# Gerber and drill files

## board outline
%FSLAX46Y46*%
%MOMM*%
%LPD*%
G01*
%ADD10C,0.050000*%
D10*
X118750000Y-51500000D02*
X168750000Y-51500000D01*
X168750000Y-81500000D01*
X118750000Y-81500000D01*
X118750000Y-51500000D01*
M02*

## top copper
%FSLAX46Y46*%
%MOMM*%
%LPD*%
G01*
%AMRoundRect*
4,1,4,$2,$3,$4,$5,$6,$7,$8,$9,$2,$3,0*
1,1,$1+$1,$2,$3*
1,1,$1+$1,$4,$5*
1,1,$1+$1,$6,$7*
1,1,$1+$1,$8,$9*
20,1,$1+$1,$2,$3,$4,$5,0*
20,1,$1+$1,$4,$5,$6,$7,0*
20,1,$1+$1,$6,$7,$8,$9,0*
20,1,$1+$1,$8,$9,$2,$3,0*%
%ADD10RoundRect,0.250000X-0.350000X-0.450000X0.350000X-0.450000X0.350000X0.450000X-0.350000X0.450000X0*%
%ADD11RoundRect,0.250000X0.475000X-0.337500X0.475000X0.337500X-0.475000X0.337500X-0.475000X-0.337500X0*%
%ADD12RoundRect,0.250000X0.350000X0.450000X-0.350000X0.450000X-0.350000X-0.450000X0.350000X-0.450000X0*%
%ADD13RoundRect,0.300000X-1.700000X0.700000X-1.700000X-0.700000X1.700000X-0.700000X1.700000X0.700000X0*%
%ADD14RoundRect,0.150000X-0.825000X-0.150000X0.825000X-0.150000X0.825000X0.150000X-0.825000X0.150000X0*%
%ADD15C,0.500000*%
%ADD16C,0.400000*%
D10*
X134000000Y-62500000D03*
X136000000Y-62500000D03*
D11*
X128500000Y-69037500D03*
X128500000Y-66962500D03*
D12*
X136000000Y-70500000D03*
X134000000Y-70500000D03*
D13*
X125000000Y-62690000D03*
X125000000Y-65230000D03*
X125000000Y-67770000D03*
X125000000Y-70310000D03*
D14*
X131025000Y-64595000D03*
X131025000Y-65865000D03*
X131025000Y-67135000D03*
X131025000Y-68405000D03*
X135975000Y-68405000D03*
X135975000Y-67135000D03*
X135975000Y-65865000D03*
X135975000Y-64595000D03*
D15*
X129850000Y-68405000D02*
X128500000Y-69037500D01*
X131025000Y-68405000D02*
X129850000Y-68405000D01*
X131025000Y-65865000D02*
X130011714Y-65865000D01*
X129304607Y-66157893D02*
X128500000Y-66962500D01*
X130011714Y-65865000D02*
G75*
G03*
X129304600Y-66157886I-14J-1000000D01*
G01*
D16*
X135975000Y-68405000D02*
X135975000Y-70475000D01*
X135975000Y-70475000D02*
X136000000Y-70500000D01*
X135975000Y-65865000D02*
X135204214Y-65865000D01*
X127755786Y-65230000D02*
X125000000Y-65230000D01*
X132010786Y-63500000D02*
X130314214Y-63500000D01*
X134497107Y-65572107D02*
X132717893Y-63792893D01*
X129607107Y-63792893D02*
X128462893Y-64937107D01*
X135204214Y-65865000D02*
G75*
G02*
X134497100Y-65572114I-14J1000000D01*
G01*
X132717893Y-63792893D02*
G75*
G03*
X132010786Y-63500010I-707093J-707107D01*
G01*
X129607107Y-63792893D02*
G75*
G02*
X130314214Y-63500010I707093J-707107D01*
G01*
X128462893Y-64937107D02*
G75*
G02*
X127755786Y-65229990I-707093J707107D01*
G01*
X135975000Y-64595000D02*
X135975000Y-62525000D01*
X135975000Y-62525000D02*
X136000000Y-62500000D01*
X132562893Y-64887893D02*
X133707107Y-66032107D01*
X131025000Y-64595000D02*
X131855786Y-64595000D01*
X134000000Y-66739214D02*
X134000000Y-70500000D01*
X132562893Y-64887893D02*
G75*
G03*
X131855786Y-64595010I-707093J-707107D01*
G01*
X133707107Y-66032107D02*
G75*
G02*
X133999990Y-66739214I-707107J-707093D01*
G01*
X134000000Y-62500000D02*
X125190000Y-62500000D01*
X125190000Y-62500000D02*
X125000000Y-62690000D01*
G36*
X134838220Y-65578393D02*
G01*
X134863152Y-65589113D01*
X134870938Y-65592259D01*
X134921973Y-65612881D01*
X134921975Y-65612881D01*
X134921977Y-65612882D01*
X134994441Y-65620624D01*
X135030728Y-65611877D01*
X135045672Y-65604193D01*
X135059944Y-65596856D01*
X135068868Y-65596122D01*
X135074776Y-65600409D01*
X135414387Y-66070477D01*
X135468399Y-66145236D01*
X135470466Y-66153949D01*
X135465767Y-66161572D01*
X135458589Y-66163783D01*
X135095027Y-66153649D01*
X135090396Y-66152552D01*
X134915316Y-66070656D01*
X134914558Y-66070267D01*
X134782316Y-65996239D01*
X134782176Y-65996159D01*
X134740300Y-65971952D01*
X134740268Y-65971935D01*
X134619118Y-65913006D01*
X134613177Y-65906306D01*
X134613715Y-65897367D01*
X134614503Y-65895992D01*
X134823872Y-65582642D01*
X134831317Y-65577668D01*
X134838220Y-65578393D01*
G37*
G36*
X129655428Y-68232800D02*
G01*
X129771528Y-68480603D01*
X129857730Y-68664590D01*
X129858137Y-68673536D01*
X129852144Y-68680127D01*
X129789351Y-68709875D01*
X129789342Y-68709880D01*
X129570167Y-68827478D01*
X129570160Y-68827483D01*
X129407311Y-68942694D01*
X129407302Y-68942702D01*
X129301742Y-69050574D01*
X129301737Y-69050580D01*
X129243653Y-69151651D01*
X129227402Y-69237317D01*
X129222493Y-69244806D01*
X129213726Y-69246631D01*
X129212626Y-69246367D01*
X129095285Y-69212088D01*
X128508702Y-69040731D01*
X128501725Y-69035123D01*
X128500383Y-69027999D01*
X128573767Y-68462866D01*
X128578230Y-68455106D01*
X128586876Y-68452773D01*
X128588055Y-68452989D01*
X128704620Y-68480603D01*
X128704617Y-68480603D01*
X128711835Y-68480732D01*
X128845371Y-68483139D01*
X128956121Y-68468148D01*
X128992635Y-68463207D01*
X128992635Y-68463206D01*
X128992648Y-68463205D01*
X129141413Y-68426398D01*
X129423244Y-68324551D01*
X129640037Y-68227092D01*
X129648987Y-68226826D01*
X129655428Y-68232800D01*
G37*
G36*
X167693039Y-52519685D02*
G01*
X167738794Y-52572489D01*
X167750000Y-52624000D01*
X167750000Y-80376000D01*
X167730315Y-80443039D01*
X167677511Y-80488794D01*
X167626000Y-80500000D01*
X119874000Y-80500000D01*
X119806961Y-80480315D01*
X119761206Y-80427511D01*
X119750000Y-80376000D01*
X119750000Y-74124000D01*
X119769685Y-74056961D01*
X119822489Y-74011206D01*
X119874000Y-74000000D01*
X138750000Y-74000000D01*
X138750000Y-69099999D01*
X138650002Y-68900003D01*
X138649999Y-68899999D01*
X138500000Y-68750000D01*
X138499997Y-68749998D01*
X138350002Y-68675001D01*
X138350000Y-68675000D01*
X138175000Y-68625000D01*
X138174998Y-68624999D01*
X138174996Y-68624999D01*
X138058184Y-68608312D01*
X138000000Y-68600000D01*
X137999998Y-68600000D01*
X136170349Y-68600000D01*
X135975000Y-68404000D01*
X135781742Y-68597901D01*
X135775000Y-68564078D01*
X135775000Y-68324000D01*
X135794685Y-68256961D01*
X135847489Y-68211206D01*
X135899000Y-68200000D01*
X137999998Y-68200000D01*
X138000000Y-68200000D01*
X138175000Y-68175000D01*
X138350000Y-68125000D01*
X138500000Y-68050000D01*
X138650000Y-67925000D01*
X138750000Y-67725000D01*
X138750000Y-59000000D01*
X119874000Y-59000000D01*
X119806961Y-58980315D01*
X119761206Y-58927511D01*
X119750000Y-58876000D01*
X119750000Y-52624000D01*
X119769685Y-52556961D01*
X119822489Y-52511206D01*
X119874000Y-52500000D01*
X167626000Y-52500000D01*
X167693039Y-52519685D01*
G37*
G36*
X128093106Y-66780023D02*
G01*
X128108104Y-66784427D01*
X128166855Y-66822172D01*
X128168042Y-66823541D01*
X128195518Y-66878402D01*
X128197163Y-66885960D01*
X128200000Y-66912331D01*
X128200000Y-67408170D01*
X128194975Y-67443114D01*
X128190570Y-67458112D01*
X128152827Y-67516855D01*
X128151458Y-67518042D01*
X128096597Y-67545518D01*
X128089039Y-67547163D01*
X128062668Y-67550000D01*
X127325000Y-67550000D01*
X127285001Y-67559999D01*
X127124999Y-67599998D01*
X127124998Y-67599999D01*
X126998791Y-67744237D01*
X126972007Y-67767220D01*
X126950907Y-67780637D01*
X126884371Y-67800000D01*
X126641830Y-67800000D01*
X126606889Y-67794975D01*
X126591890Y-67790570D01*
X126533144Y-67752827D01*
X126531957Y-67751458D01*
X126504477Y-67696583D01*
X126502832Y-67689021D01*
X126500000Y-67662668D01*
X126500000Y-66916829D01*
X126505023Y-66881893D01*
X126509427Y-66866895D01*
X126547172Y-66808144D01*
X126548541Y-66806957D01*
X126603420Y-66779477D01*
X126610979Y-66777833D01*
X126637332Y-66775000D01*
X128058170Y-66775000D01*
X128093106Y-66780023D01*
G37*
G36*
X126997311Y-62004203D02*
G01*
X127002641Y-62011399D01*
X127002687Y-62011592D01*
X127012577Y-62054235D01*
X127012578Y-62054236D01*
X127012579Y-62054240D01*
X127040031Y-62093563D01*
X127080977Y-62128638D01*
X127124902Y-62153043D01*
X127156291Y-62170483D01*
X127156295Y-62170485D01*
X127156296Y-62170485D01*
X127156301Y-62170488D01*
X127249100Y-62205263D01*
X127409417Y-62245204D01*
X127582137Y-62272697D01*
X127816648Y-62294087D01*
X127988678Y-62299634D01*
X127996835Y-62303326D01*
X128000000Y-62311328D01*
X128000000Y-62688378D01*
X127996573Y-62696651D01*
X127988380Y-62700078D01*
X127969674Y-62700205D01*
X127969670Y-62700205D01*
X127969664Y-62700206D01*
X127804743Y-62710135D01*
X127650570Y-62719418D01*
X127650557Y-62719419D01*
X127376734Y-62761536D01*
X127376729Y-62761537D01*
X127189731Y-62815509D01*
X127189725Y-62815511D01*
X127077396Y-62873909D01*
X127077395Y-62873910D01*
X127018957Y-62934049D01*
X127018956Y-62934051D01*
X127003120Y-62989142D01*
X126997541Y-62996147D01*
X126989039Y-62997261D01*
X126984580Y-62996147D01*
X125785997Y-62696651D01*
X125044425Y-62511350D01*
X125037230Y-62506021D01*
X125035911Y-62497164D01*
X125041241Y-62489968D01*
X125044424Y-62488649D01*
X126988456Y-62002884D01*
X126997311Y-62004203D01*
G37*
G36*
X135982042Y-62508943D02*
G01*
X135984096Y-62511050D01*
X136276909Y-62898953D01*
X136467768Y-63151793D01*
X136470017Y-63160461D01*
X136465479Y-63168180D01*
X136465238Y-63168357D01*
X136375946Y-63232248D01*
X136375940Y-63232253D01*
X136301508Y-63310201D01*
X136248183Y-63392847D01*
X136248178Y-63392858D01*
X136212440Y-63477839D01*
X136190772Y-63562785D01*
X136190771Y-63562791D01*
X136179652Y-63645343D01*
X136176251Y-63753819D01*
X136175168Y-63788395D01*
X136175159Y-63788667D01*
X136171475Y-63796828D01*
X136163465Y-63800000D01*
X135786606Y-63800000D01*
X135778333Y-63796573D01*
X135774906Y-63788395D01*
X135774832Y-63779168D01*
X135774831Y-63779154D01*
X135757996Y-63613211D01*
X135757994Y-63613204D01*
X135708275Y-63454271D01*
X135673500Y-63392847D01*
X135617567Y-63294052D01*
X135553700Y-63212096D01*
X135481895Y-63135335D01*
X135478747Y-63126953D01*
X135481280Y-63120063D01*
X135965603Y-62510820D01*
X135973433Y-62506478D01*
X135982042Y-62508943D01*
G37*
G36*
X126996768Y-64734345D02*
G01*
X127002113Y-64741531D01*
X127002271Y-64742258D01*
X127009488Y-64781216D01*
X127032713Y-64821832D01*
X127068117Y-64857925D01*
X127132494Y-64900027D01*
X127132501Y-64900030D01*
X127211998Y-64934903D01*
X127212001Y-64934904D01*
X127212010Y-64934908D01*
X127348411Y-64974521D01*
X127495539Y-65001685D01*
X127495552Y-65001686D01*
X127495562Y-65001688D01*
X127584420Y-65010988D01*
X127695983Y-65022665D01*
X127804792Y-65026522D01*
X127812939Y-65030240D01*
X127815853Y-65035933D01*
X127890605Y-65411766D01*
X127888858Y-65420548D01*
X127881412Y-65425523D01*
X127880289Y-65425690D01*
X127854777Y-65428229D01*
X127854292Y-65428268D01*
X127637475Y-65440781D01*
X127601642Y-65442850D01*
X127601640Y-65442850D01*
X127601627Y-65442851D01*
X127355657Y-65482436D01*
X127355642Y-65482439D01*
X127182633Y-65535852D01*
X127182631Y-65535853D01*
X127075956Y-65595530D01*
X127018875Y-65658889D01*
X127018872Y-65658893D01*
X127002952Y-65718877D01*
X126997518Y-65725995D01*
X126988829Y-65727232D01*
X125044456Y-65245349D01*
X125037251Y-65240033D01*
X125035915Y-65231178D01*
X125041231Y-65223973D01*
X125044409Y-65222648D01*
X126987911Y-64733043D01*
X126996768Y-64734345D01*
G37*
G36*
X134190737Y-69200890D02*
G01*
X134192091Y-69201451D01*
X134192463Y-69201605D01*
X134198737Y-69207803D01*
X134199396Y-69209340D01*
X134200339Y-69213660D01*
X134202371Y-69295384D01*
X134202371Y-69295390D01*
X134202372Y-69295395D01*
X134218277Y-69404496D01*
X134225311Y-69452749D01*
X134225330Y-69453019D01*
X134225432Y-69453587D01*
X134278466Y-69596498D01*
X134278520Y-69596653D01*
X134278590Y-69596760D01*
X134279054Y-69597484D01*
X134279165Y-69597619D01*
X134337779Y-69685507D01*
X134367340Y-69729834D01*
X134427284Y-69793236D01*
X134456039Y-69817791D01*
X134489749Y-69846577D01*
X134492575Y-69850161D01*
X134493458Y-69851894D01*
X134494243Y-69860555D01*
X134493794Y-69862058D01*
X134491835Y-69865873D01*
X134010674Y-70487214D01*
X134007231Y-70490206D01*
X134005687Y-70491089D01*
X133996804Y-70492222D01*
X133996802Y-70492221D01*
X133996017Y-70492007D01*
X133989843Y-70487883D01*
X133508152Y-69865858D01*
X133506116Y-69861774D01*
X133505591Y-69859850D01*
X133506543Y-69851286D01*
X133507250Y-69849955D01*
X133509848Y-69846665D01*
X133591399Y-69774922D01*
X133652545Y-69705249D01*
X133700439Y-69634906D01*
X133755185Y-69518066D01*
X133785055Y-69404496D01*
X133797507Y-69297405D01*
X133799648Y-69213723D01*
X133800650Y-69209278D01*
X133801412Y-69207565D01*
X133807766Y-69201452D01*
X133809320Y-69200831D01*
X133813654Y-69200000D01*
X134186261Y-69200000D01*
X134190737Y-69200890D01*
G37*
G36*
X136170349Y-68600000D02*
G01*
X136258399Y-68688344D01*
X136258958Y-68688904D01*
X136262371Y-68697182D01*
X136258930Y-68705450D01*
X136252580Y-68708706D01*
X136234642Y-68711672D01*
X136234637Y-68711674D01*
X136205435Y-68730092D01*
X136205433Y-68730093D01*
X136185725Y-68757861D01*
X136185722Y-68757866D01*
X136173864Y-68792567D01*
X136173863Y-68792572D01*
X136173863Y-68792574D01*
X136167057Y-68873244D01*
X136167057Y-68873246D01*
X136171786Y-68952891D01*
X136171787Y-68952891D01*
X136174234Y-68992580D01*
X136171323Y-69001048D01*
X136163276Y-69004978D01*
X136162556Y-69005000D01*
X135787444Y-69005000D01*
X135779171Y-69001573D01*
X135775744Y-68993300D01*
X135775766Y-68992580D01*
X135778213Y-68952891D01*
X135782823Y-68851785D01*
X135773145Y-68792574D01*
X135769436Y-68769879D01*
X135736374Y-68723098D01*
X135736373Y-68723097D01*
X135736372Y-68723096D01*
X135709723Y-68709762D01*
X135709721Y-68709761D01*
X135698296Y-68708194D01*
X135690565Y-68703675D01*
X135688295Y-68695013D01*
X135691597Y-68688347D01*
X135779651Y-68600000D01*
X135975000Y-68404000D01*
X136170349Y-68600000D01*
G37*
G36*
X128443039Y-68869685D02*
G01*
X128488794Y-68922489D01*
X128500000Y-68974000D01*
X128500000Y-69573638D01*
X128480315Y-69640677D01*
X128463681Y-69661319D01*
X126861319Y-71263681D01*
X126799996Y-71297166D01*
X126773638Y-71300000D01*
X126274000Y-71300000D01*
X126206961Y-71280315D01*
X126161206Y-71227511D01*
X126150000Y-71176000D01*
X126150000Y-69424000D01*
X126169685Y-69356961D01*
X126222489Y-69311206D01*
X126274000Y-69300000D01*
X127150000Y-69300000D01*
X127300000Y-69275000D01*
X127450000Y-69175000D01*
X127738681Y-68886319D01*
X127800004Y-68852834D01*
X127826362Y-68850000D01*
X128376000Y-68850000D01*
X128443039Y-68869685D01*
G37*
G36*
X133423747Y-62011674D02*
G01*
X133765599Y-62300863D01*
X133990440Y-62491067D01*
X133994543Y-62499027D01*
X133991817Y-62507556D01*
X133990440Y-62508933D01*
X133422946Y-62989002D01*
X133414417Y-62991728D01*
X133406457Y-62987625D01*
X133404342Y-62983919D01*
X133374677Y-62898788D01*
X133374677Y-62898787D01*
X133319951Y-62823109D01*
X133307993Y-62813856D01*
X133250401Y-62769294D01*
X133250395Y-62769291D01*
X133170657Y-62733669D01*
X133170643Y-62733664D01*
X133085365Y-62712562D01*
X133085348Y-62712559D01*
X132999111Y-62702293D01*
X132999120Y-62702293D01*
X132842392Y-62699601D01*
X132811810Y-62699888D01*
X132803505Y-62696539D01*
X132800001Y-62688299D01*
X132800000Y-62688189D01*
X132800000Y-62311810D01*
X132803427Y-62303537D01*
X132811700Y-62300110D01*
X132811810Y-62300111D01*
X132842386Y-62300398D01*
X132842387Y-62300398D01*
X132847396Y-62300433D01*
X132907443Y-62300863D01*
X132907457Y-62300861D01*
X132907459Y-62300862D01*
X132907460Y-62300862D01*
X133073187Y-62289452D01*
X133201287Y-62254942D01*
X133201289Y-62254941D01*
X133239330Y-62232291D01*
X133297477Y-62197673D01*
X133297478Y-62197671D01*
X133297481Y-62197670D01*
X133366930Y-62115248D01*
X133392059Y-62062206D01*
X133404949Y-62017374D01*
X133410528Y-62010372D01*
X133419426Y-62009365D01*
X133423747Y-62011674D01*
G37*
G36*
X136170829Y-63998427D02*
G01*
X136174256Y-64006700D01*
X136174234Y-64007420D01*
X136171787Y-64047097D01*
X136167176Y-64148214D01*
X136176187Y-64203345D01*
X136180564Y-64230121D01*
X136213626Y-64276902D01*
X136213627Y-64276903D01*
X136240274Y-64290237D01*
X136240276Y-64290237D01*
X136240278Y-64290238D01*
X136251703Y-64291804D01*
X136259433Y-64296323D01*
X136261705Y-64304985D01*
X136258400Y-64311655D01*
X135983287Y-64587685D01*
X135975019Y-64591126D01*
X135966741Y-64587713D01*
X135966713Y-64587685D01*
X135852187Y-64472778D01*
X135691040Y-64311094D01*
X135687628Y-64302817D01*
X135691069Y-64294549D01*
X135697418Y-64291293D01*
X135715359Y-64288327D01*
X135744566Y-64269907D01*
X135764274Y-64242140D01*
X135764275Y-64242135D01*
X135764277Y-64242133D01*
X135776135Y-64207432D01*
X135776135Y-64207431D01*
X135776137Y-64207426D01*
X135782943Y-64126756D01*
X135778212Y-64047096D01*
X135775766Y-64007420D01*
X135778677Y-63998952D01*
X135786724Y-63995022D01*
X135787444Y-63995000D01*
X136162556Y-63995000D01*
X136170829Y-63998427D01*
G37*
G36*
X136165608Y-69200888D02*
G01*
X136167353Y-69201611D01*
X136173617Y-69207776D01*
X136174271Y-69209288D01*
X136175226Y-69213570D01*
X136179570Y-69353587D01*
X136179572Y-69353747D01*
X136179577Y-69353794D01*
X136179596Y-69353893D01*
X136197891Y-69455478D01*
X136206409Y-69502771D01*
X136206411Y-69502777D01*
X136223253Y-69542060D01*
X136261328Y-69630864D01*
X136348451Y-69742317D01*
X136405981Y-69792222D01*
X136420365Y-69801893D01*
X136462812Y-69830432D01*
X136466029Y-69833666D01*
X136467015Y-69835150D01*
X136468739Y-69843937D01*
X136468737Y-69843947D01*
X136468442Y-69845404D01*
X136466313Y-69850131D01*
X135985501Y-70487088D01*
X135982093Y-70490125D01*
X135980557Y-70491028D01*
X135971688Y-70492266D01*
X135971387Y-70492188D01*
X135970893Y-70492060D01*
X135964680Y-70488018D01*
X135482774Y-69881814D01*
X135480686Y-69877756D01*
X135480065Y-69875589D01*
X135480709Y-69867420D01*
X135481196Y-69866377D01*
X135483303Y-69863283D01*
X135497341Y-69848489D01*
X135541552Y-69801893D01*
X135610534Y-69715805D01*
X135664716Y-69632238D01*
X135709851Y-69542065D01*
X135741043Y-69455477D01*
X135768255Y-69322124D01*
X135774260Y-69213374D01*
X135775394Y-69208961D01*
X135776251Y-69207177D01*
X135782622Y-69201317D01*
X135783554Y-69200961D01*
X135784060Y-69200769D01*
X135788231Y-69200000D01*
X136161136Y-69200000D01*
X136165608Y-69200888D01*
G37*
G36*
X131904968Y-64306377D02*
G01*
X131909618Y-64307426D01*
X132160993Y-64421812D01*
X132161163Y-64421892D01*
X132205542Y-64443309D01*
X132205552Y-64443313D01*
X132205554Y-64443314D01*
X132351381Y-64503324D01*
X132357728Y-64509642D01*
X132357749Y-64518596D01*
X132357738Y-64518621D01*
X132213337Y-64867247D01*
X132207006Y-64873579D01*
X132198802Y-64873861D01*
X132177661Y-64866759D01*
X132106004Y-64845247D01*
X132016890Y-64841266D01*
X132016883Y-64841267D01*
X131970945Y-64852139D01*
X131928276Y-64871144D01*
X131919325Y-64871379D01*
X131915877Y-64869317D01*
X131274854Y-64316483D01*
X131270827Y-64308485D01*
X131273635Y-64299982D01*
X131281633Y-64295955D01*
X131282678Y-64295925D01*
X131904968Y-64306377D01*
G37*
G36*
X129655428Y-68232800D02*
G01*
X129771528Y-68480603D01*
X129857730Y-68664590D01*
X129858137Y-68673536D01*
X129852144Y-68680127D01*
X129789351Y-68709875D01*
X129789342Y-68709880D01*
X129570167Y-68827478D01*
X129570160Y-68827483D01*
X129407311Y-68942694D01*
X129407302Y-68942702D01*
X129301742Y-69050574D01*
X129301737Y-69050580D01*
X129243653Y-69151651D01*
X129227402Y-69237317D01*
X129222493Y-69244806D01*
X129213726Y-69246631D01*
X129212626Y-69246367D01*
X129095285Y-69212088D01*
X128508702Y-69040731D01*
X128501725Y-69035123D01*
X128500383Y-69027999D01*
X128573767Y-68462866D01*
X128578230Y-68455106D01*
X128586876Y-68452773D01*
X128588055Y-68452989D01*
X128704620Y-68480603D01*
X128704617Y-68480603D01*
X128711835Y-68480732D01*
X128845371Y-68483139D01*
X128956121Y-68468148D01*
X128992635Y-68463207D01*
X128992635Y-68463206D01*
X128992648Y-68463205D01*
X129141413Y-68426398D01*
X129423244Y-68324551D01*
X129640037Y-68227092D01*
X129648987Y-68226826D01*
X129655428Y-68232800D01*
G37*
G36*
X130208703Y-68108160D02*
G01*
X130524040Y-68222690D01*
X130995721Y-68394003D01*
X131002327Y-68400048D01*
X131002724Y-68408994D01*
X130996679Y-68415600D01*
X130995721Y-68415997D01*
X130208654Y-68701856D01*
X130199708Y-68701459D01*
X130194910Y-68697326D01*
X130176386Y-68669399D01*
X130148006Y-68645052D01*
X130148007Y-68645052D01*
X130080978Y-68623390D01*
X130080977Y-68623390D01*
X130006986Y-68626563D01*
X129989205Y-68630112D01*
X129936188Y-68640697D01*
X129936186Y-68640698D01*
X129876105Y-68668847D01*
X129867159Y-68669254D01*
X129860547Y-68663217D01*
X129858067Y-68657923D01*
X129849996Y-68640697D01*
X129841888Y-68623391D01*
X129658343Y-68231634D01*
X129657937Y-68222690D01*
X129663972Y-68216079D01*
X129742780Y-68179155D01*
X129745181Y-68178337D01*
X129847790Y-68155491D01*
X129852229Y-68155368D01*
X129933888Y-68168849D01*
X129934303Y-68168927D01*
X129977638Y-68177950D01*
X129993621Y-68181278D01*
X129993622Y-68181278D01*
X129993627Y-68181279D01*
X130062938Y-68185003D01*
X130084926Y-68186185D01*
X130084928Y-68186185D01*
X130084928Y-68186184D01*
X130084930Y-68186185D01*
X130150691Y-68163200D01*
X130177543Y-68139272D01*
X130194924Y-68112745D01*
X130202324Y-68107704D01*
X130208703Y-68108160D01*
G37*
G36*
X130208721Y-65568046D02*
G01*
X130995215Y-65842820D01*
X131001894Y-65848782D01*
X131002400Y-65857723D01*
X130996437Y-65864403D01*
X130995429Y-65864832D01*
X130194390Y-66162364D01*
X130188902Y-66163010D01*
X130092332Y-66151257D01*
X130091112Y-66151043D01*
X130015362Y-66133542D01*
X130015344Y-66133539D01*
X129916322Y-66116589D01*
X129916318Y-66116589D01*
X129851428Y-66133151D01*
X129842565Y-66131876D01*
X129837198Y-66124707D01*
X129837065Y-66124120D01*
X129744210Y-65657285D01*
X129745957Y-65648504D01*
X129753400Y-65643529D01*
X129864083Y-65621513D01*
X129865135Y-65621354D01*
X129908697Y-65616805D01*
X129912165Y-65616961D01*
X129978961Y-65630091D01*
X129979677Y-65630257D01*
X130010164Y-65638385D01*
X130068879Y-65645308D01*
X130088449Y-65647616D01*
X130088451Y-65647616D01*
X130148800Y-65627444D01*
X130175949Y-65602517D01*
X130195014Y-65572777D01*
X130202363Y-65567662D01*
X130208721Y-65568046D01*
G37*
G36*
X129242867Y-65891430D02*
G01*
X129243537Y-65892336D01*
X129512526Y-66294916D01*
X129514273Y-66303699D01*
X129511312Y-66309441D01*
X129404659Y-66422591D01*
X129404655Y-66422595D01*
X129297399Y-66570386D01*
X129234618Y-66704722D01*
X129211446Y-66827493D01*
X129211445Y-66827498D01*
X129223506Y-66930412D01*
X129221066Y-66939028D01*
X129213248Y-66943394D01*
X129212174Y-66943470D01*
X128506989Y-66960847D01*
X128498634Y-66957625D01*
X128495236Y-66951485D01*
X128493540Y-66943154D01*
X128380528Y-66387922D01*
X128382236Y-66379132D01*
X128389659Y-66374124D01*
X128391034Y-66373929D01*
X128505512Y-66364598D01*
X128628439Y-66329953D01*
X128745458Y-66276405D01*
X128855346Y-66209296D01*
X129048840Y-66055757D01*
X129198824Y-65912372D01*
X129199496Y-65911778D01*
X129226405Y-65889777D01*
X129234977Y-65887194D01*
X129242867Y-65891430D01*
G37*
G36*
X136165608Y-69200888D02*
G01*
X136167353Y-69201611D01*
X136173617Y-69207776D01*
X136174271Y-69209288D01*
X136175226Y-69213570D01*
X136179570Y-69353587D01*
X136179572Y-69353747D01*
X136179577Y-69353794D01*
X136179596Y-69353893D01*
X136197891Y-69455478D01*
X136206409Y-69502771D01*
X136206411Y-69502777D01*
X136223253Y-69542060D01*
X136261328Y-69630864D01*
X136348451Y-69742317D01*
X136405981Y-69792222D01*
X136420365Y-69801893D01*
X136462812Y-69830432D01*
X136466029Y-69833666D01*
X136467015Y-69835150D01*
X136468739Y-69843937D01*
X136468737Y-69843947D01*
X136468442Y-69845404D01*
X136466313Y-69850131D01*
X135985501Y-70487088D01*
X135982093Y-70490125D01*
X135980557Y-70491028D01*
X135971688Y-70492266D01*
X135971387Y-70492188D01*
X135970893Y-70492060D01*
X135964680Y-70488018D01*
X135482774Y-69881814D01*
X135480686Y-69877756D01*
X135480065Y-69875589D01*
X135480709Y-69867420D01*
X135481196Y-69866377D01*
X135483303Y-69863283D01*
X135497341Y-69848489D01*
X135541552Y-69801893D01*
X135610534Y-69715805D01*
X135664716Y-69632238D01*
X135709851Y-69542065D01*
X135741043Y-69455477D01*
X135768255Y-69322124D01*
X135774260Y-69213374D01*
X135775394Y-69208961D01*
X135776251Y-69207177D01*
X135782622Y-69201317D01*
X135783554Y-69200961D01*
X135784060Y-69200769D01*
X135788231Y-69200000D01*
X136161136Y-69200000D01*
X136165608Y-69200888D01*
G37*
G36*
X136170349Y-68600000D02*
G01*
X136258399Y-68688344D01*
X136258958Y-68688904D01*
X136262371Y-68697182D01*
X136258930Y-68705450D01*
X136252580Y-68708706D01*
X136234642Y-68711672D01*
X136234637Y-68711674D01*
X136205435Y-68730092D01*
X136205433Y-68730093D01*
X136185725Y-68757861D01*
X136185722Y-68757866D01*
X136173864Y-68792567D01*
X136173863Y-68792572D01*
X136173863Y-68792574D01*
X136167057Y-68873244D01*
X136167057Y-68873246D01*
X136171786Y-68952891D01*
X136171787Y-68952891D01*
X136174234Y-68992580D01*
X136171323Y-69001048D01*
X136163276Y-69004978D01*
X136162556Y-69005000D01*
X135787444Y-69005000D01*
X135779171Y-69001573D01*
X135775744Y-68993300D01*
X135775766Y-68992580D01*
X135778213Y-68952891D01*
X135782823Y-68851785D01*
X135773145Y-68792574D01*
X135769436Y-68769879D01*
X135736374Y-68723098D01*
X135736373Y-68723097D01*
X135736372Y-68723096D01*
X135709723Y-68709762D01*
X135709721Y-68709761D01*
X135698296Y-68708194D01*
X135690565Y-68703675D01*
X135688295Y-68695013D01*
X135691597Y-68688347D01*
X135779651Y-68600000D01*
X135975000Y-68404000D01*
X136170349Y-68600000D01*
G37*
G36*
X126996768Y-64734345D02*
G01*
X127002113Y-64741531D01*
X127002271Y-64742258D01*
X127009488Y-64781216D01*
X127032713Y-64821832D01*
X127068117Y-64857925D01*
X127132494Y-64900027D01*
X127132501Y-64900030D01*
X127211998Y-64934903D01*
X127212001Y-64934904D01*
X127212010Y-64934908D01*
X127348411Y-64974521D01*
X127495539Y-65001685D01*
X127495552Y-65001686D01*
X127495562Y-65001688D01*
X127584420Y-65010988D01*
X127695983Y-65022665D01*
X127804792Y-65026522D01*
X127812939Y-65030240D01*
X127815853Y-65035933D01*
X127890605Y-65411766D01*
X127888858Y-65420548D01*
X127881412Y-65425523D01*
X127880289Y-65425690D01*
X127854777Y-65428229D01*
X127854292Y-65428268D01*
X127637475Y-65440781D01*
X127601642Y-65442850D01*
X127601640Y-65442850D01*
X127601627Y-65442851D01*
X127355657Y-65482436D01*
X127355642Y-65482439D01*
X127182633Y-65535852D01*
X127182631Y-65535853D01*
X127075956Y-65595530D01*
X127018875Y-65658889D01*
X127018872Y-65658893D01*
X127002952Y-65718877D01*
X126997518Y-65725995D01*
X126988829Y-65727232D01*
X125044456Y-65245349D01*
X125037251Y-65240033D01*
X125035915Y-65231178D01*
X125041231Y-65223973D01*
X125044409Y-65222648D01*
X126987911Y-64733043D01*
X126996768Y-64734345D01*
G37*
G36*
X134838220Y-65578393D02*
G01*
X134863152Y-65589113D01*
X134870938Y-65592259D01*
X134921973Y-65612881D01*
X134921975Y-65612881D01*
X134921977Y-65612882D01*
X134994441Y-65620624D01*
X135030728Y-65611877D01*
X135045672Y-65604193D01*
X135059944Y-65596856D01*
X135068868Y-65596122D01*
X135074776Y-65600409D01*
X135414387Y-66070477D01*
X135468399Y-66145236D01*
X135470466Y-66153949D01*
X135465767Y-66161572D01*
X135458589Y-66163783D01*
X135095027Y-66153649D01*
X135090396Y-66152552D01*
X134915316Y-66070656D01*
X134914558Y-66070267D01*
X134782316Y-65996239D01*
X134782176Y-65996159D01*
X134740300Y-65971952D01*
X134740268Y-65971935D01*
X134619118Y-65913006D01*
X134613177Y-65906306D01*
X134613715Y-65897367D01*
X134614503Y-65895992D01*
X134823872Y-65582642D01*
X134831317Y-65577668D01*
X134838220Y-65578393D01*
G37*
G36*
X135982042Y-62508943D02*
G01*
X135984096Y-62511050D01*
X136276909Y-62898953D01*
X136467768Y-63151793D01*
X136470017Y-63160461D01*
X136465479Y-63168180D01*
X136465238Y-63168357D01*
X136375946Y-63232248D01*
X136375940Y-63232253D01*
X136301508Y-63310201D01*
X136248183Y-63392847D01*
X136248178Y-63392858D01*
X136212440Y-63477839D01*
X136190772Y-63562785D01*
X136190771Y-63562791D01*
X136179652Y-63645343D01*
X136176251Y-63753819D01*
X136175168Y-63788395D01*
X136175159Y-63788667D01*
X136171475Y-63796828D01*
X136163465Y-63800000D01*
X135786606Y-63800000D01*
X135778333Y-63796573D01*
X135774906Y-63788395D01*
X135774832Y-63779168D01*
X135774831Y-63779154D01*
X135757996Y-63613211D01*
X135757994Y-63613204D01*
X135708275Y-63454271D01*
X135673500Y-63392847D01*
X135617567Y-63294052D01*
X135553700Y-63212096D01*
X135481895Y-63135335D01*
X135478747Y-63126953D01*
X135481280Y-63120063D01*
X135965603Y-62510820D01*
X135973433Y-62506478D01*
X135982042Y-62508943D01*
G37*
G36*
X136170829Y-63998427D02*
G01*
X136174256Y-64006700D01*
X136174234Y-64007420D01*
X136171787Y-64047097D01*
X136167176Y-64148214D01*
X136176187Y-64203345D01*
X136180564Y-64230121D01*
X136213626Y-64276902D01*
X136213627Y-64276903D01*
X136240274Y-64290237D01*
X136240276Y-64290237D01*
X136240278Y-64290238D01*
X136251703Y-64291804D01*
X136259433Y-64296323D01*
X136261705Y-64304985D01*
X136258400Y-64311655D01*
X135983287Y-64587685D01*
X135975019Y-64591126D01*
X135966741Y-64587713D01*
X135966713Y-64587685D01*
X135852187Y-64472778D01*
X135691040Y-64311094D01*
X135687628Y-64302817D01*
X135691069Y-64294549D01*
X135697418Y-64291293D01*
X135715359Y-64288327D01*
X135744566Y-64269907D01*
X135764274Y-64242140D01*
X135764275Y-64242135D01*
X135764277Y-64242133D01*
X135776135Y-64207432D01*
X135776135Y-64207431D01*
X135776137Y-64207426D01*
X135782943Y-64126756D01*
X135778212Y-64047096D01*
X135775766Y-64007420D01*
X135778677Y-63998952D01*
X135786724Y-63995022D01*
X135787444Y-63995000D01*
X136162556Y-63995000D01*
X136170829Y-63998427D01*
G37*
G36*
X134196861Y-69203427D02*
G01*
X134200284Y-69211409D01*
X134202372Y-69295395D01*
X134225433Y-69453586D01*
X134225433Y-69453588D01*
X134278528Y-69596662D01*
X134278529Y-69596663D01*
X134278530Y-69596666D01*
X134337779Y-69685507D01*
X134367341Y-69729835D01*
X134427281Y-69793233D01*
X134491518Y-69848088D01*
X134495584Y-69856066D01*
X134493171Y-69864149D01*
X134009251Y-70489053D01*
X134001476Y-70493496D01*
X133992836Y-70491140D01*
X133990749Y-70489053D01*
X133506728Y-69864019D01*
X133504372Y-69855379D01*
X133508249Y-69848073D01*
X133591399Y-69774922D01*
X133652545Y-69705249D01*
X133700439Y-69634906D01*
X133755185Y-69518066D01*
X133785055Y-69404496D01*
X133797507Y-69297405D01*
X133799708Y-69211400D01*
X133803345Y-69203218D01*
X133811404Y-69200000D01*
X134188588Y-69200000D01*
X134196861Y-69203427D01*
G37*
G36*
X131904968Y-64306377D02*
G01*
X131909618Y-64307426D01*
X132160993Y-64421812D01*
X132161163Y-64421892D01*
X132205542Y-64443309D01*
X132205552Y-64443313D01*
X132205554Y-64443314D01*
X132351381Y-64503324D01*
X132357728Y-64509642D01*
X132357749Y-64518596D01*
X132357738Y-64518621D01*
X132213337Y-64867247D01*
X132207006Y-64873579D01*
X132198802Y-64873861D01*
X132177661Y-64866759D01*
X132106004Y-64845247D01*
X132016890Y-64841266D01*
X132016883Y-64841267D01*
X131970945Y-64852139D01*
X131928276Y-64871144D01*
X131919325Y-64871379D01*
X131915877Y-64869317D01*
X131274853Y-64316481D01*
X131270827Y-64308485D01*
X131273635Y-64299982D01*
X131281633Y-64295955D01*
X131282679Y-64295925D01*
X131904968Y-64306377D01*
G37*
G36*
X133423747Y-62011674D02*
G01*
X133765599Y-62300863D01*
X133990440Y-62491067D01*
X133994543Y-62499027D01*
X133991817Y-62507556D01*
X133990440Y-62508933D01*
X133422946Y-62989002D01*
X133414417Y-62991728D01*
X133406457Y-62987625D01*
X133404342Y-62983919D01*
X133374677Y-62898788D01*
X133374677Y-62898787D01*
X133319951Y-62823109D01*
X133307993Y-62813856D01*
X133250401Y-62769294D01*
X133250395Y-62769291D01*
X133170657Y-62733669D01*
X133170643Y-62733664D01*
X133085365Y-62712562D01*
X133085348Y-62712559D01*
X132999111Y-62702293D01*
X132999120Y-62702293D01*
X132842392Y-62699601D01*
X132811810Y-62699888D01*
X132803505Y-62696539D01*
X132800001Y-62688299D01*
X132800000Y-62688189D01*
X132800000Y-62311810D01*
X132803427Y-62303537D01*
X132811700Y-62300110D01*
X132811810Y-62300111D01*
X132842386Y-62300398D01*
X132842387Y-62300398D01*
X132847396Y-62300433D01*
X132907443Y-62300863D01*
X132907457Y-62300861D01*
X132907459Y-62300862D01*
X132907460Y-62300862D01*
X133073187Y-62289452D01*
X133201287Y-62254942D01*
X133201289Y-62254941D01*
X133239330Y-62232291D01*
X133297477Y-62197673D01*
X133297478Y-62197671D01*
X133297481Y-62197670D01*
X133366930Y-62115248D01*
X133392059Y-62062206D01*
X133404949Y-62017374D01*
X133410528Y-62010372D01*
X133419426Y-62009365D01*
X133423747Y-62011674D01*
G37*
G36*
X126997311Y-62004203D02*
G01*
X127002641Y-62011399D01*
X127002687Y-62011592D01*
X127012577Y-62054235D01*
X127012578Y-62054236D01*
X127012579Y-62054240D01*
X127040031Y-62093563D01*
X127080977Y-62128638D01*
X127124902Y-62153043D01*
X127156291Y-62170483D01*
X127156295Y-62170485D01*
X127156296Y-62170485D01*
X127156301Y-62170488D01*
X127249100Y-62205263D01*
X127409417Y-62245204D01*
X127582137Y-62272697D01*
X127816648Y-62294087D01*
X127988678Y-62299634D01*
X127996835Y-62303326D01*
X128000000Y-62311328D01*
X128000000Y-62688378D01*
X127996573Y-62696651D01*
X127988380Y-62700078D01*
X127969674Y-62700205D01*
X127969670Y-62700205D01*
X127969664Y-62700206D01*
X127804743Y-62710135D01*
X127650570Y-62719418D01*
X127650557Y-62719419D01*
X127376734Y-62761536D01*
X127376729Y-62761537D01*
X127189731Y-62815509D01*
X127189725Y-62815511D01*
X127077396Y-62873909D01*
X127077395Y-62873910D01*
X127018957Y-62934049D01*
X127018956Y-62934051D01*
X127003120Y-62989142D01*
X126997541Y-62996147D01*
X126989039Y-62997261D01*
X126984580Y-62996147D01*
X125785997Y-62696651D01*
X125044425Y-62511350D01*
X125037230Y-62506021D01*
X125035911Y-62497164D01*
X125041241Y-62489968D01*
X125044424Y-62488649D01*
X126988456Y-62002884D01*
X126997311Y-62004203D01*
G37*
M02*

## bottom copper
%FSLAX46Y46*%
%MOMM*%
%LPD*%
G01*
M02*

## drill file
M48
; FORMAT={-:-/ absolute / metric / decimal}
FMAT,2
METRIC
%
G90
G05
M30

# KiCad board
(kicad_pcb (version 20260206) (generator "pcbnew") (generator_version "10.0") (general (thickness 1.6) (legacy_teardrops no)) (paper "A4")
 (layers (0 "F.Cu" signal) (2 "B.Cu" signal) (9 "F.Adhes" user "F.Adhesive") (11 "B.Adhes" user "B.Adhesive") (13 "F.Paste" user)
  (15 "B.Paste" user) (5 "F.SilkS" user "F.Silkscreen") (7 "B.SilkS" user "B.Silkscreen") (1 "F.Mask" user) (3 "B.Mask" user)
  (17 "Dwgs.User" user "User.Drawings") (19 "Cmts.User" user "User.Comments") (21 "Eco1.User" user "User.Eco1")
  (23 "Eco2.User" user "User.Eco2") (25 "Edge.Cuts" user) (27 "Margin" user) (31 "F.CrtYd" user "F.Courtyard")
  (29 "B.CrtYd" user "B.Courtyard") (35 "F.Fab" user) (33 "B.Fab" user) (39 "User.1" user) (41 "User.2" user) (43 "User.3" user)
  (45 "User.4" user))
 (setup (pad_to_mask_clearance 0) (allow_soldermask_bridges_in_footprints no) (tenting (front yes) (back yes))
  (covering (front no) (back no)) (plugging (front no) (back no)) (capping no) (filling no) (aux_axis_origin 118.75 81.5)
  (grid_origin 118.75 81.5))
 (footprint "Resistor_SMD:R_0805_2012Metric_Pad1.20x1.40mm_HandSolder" (layer "F.Cu") (at 135 62.5)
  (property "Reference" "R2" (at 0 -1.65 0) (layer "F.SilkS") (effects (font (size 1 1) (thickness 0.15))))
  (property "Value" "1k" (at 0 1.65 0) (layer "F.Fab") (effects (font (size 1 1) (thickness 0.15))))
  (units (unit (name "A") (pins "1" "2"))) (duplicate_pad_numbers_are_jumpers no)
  (pad "1" smd roundrect (at -1 0) (size 1.2 1.4) (layers "F.Cu" "F.Mask" "F.Paste") (roundrect_rratio 0.208333) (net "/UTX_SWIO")
   (teardrops (best_length_ratio 0.5) (max_length 1) (best_width_ratio 1) (max_width 1) (curved_edges yes) (filter_ratio 0.9) (enabled yes)
    (allow_two_segments yes) (prefer_zone_connections yes)))
  (pad "2" smd roundrect (at 1 0) (size 1.2 1.4) (layers "F.Cu" "F.Mask" "F.Paste") (roundrect_rratio 0.208333)
   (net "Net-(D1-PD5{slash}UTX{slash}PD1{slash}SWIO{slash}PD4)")
   (teardrops (best_length_ratio 0.5) (max_length 1) (best_width_ratio 1) (max_width 1) (curved_edges yes) (filter_ratio 0.9) (enabled yes)
    (allow_two_segments yes) (prefer_zone_connections yes))))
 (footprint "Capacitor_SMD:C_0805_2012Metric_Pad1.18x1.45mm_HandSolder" (layer "F.Cu") (at 128.5 68 90)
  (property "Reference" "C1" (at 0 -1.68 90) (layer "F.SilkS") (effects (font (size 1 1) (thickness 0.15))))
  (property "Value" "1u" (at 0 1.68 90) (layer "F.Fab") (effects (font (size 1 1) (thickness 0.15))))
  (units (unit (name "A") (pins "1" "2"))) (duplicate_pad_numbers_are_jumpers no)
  (pad "1" smd roundrect (at -1.0375 0 90) (size 1.175 1.45) (layers "F.Cu" "F.Mask" "F.Paste") (roundrect_rratio 0.212766) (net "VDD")
   (teardrops (best_length_ratio 0.5) (max_length 1) (best_width_ratio 1) (max_width 1) (curved_edges yes) (filter_ratio 0.9) (enabled yes)
    (allow_two_segments yes) (prefer_zone_connections yes)))
  (pad "2" smd roundrect (at 1.0375 0 90) (size 1.175 1.45) (layers "F.Cu" "F.Mask" "F.Paste") (roundrect_rratio 0.212766) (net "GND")
   (teardrops (best_length_ratio 0.5) (max_length 1) (best_width_ratio 1) (max_width 1) (curved_edges yes) (filter_ratio 0.9) (enabled yes)
    (allow_two_segments yes) (prefer_zone_connections yes))))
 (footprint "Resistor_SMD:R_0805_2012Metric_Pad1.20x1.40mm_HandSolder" (layer "F.Cu") (at 135 70.5 180)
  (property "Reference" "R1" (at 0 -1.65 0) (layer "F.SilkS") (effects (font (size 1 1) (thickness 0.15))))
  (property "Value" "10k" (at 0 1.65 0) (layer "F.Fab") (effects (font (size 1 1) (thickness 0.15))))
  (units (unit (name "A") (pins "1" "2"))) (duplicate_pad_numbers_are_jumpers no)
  (pad "1" smd roundrect (at -1 0 180) (size 1.2 1.4) (layers "F.Cu" "F.Mask" "F.Paste") (roundrect_rratio 0.208333) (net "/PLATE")
   (teardrops (best_length_ratio 0.5) (max_length 1) (best_width_ratio 1) (max_width 1) (curved_edges yes) (filter_ratio 0.9) (enabled yes)
    (allow_two_segments yes) (prefer_zone_connections yes)))
  (pad "2" smd roundrect (at 1 0 180) (size 1.2 1.4) (layers "F.Cu" "F.Mask" "F.Paste") (roundrect_rratio 0.208333)
   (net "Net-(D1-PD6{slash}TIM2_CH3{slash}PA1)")
   (teardrops (best_length_ratio 0.5) (max_length 1) (best_width_ratio 1) (max_width 1) (curved_edges yes) (filter_ratio 0.9) (enabled yes)
    (allow_two_segments yes) (prefer_zone_connections yes))))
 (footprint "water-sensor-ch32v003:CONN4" (layer "F.Cu") (at 125 62.69 -90)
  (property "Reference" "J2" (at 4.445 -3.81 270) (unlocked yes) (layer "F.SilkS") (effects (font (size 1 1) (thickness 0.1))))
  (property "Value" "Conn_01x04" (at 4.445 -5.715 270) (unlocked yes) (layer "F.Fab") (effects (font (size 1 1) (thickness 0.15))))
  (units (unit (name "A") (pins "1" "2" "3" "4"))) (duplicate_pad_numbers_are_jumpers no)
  (pad "1" smd roundrect (at 0 0 270) (size 2 4) (layers "F.Cu" "F.Mask" "F.Paste") (roundrect_rratio 0.15) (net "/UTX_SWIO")
   (teardrops (best_length_ratio 0.5) (max_length 1) (best_width_ratio 1) (max_width 1) (curved_edges yes) (filter_ratio 0.9) (enabled yes)
    (allow_two_segments yes) (prefer_zone_connections yes)))
  (pad "2" smd roundrect (at 2.54 0 270) (size 2 4) (layers "F.Cu" "F.Mask" "F.Paste") (roundrect_rratio 0.15) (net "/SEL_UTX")
   (teardrops (best_length_ratio 0.5) (max_length 1) (best_width_ratio 1) (max_width 1) (curved_edges yes) (filter_ratio 0.9) (enabled yes)
    (allow_two_segments yes) (prefer_zone_connections yes)))
  (pad "3" smd roundrect (at 5.08 0 270) (size 2 4) (layers "F.Cu" "F.Mask" "F.Paste") (roundrect_rratio 0.15) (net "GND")
   (teardrops (best_length_ratio 0.5) (max_length 1) (best_width_ratio 1) (max_width 1) (curved_edges yes) (filter_ratio 0.9) (enabled yes)
    (allow_two_segments yes) (prefer_zone_connections yes)))
  (pad "4" smd roundrect (at 7.62 0 270) (size 2 4) (layers "F.Cu" "F.Mask" "F.Paste") (roundrect_rratio 0.15) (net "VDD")
   (teardrops (best_length_ratio 0.5) (max_length 1) (best_width_ratio 1) (max_width 1) (curved_edges yes) (filter_ratio 0.9) (enabled yes)
    (allow_two_segments yes) (prefer_zone_connections yes))))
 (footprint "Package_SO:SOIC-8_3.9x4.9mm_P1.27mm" (layer "F.Cu") (at 133.5 66.5)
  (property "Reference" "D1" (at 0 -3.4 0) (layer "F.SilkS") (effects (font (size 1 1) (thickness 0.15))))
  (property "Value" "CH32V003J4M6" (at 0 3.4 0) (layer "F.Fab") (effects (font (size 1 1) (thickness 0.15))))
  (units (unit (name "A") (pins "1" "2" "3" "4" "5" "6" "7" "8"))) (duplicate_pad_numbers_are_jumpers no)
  (pad "1" smd roundrect (at -2.475 -1.905) (size 1.95 0.6) (layers "F.Cu" "F.Mask" "F.Paste") (roundrect_rratio 0.25)
   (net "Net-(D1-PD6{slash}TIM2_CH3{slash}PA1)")
   (teardrops (best_length_ratio 0.5) (max_length 1) (best_width_ratio 1) (max_width 1) (curved_edges yes) (filter_ratio 0.9) (enabled yes)
    (allow_two_segments yes) (prefer_zone_connections yes)))
  (pad "2" smd roundrect (at -2.475 -0.635) (size 1.95 0.6) (layers "F.Cu" "F.Mask" "F.Paste") (roundrect_rratio 0.25) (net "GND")
   (teardrops (best_length_ratio 0.5) (max_length 1) (best_width_ratio 1) (max_width 1) (curved_edges yes) (filter_ratio 0.9) (enabled yes)
    (allow_two_segments yes) (prefer_zone_connections yes)))
  (pad "3" smd roundrect (at -2.475 0.635) (size 1.95 0.6) (layers "F.Cu" "F.Mask" "F.Paste") (roundrect_rratio 0.25)
   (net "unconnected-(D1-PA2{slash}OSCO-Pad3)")
   (teardrops (best_length_ratio 0.5) (max_length 1) (best_width_ratio 1) (max_width 1) (curved_edges yes) (filter_ratio 0.9) (enabled yes)
    (allow_two_segments yes) (prefer_zone_connections yes)))
  (pad "4" smd roundrect (at -2.475 1.905) (size 1.95 0.6) (layers "F.Cu" "F.Mask" "F.Paste") (roundrect_rratio 0.25) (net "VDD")
   (teardrops (best_length_ratio 0.5) (max_length 1) (best_width_ratio 1) (max_width 1) (curved_edges yes) (filter_ratio 0.9) (enabled yes)
    (allow_two_segments yes) (prefer_zone_connections yes)))
  (pad "5" smd roundrect (at 2.475 1.905) (size 1.95 0.6) (layers "F.Cu" "F.Mask" "F.Paste") (roundrect_rratio 0.25) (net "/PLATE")
   (teardrops (best_length_ratio 0.5) (max_length 1) (best_width_ratio 1) (max_width 1) (curved_edges yes) (filter_ratio 0.9) (enabled yes)
    (allow_two_segments yes) (prefer_zone_connections yes)))
  (pad "6" smd roundrect (at 2.475 0.635) (size 1.95 0.6) (layers "F.Cu" "F.Mask" "F.Paste") (roundrect_rratio 0.25)
   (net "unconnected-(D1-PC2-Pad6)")
   (teardrops (best_length_ratio 0.5) (max_length 1) (best_width_ratio 1) (max_width 1) (curved_edges yes) (filter_ratio 0.9) (enabled yes)
    (allow_two_segments yes) (prefer_zone_connections yes)))
  (pad "7" smd roundrect (at 2.475 -0.635) (size 1.95 0.6) (layers "F.Cu" "F.Mask" "F.Paste") (roundrect_rratio 0.25) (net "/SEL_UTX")
   (teardrops (best_length_ratio 0.5) (max_length 1) (best_width_ratio 1) (max_width 1) (curved_edges yes) (filter_ratio 0.9) (enabled yes)
    (allow_two_segments yes) (prefer_zone_connections yes)))
  (pad "8" smd roundrect (at 2.475 -1.905) (size 1.95 0.6) (layers "F.Cu" "F.Mask" "F.Paste") (roundrect_rratio 0.25)
   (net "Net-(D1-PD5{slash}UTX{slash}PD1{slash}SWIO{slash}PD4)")
   (teardrops (best_length_ratio 0.5) (max_length 1) (best_width_ratio 1) (max_width 1) (curved_edges yes) (filter_ratio 0.9) (enabled yes)
    (allow_two_segments yes) (prefer_zone_connections yes))))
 (gr_rect (start 118.75 51.5) (end 168.75 81.5) (stroke (width 0.05) (type default)) (fill no) (layer "Edge.Cuts"))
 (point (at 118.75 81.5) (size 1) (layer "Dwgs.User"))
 (segment (start 129.85 68.405) (end 128.5 69.0375) (width 0.5) (layer "F.Cu") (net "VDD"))
 (segment (start 131.025 68.405) (end 129.85 68.405) (width 0.5) (layer "F.Cu") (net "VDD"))
 (segment (start 131.025 65.865) (end 130.011714 65.865) (width 0.5) (layer "F.Cu") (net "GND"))
 (segment (start 129.304607 66.157893) (end 128.5 66.9625) (width 0.5) (layer "F.Cu") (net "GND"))
 (arc (start 130.011714 65.865) (mid 129.629031 65.94112) (end 129.304607 66.157893) (width 0.5) (layer "F.Cu") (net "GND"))
 (segment (start 135.975 68.405) (end 135.975 70.475) (width 0.4) (layer "F.Cu") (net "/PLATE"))
 (segment (start 135.975 70.475) (end 136 70.5) (width 0.4) (layer "F.Cu") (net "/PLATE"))
 (segment (start 135.975 65.865) (end 135.204214 65.865) (width 0.4) (layer "F.Cu") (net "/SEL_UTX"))
 (segment (start 127.755786 65.23) (end 125 65.23) (width 0.4) (layer "F.Cu") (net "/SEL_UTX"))
 (segment (start 132.010786 63.5) (end 130.314214 63.5) (width 0.4) (layer "F.Cu") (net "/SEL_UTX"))
 (segment (start 134.497107 65.572107) (end 132.717893 63.792893) (width 0.4) (layer "F.Cu") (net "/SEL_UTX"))
 (segment (start 129.607107 63.792893) (end 128.462893 64.937107) (width 0.4) (layer "F.Cu") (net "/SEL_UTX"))
 (arc (start 135.204214 65.865) (mid 134.821531 65.78888) (end 134.497107 65.572107) (width 0.4) (layer "F.Cu") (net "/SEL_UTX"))
 (arc (start 132.717893 63.792893) (mid 132.39347 63.57612) (end 132.010786 63.5) (width 0.4) (layer "F.Cu") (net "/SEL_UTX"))
 (arc (start 129.607107 63.792893) (mid 129.93153 63.57612) (end 130.314214 63.5) (width 0.4) (layer "F.Cu") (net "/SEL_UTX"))
 (arc (start 128.462893 64.937107) (mid 128.13847 65.15388) (end 127.755786 65.23) (width 0.4) (layer "F.Cu") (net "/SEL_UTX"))
 (segment (start 135.975 64.595) (end 135.975 62.525) (width 0.4) (layer "F.Cu")
  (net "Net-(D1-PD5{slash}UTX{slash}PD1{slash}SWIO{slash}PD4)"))
 (segment (start 135.975 62.525) (end 136 62.5) (width 0.4) (layer "F.Cu") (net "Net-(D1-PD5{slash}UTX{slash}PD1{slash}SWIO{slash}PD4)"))
 (segment (start 132.562893 64.887893) (end 133.707107 66.032107) (width 0.4) (layer "F.Cu") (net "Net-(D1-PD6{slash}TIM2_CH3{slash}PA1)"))
 (segment (start 131.025 64.595) (end 131.855786 64.595) (width 0.4) (layer "F.Cu") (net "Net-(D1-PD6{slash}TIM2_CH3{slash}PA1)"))
 (segment (start 134 66.739214) (end 134 70.5) (width 0.4) (layer "F.Cu") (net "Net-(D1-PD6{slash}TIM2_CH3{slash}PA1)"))
 (arc (start 132.562893 64.887893) (mid 132.23847 64.67112) (end 131.855786 64.595) (width 0.4) (layer "F.Cu")
  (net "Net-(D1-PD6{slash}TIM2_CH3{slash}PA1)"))
 (arc (start 133.707107 66.032107) (mid 133.92388 66.35653) (end 134 66.739214) (width 0.4) (layer "F.Cu")
  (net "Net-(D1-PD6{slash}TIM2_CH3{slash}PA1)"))
 (segment (start 134 62.5) (end 125.19 62.5) (width 0.4) (layer "F.Cu") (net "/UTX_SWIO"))
 (segment (start 125.19 62.5) (end 125 62.69) (width 0.4) (layer "F.Cu") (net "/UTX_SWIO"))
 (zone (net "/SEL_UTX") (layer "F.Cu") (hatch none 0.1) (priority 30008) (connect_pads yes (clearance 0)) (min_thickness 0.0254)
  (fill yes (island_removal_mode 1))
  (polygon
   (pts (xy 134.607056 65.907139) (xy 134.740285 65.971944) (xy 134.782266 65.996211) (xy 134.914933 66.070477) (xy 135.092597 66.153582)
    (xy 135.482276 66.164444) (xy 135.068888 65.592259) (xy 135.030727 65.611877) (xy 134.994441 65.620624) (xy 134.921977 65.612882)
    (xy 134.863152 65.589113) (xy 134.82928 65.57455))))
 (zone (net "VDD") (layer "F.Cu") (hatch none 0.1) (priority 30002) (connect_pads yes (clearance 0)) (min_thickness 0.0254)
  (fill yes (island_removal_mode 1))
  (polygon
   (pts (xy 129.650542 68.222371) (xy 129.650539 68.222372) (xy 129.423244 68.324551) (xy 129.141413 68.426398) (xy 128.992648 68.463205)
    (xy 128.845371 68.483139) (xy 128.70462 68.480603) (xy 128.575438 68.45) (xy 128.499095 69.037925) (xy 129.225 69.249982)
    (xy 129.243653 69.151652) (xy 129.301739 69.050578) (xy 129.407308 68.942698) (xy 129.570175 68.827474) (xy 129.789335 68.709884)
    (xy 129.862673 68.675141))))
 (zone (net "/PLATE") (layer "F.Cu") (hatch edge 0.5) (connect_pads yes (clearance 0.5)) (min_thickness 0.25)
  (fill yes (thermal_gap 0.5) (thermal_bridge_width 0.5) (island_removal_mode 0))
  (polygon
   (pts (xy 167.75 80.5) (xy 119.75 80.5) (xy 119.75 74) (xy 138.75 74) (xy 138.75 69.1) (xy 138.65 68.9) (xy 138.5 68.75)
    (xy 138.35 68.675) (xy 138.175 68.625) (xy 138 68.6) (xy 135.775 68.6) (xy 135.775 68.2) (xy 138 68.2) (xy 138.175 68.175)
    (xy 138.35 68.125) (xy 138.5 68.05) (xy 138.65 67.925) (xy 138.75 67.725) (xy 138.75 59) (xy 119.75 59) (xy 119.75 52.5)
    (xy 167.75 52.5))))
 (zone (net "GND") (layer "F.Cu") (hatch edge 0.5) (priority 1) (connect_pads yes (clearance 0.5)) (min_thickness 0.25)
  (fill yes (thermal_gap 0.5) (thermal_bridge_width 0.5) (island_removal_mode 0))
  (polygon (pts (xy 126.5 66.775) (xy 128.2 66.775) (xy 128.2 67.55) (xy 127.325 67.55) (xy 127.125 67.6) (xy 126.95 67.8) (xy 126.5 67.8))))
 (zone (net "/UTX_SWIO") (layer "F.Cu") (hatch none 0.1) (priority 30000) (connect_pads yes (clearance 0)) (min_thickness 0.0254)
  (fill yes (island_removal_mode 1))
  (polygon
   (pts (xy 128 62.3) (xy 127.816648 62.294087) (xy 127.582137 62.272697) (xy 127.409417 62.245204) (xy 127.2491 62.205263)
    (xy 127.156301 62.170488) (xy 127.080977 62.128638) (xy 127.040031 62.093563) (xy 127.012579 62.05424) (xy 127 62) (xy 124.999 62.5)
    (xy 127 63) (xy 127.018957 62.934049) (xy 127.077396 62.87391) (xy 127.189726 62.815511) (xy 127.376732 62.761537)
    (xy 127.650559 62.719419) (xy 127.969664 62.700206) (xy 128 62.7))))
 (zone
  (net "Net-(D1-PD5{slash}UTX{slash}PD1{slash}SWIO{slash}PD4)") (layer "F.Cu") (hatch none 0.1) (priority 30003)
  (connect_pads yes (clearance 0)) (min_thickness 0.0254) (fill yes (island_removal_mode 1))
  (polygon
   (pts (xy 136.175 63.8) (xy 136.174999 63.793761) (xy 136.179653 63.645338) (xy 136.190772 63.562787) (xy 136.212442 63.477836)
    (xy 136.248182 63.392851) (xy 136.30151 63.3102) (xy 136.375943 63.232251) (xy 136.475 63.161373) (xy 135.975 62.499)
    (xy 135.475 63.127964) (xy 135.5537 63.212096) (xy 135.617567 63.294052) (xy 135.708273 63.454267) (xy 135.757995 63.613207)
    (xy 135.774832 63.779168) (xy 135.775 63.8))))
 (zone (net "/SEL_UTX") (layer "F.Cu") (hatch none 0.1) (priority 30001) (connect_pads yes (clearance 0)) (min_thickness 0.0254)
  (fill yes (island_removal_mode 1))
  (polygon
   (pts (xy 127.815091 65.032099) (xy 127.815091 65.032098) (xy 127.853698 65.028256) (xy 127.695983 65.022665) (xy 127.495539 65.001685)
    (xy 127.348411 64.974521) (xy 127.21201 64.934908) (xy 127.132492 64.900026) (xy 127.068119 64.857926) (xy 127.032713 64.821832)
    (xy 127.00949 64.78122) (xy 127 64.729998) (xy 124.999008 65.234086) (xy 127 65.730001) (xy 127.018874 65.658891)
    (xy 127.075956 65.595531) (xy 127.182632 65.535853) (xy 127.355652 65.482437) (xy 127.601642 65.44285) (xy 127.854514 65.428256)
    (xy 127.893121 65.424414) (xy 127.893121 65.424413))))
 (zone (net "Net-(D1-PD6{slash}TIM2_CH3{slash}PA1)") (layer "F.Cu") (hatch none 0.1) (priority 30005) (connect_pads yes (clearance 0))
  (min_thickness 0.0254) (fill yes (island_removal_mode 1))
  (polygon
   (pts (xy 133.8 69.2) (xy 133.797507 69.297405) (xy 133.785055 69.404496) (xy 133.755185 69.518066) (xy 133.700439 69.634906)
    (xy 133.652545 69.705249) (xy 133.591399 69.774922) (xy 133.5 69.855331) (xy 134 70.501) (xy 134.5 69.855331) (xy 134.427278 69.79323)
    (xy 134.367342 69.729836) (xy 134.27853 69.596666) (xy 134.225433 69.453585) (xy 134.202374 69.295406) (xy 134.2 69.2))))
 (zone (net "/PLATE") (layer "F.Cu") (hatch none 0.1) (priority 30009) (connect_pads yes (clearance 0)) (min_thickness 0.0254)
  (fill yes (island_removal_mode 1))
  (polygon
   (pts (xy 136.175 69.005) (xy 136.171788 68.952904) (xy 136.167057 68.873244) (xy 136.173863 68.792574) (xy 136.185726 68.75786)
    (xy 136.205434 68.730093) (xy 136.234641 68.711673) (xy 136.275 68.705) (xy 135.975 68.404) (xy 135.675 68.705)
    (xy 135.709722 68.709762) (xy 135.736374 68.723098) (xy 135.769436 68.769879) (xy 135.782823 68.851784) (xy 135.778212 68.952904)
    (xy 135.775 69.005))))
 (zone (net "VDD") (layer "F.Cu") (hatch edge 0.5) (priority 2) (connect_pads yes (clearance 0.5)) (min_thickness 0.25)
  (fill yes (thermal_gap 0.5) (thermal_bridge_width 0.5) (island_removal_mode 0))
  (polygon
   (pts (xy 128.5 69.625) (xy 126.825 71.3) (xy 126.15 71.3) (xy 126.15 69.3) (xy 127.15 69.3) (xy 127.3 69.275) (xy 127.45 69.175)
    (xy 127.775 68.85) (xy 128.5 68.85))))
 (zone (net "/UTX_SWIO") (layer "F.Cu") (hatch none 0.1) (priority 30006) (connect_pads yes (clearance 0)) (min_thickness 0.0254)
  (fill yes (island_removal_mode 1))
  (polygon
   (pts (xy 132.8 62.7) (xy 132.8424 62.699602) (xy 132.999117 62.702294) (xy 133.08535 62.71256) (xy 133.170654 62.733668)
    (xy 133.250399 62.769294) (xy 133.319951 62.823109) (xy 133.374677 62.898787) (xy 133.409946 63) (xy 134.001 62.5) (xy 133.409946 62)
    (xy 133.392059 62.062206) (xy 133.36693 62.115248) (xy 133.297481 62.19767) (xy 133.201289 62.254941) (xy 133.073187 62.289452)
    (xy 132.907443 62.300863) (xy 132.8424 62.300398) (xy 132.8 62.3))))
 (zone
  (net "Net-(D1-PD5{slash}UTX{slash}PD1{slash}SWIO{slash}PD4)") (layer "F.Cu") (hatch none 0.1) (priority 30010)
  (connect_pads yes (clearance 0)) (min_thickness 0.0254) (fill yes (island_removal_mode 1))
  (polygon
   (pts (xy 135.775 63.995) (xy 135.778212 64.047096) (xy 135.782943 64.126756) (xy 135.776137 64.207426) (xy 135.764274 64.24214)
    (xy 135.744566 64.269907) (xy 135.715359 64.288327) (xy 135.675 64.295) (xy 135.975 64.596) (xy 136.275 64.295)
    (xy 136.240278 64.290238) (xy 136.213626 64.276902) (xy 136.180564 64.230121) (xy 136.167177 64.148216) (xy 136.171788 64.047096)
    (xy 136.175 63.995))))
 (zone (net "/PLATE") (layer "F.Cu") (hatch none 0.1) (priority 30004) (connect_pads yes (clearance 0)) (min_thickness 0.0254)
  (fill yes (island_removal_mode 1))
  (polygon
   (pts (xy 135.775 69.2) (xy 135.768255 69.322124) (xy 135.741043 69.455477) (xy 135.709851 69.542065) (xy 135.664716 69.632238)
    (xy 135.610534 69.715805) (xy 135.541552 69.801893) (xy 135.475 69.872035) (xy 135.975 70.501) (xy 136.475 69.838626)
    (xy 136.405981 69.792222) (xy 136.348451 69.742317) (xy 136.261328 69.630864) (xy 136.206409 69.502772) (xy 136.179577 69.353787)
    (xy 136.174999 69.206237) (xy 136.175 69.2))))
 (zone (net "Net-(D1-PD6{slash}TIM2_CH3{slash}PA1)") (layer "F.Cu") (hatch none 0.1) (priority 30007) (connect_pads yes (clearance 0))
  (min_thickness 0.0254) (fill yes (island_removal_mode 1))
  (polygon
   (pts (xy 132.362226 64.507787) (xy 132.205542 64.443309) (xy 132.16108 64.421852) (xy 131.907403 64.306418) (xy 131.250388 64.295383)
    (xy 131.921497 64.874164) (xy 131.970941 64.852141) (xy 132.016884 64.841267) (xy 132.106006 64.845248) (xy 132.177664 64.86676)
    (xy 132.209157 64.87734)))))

